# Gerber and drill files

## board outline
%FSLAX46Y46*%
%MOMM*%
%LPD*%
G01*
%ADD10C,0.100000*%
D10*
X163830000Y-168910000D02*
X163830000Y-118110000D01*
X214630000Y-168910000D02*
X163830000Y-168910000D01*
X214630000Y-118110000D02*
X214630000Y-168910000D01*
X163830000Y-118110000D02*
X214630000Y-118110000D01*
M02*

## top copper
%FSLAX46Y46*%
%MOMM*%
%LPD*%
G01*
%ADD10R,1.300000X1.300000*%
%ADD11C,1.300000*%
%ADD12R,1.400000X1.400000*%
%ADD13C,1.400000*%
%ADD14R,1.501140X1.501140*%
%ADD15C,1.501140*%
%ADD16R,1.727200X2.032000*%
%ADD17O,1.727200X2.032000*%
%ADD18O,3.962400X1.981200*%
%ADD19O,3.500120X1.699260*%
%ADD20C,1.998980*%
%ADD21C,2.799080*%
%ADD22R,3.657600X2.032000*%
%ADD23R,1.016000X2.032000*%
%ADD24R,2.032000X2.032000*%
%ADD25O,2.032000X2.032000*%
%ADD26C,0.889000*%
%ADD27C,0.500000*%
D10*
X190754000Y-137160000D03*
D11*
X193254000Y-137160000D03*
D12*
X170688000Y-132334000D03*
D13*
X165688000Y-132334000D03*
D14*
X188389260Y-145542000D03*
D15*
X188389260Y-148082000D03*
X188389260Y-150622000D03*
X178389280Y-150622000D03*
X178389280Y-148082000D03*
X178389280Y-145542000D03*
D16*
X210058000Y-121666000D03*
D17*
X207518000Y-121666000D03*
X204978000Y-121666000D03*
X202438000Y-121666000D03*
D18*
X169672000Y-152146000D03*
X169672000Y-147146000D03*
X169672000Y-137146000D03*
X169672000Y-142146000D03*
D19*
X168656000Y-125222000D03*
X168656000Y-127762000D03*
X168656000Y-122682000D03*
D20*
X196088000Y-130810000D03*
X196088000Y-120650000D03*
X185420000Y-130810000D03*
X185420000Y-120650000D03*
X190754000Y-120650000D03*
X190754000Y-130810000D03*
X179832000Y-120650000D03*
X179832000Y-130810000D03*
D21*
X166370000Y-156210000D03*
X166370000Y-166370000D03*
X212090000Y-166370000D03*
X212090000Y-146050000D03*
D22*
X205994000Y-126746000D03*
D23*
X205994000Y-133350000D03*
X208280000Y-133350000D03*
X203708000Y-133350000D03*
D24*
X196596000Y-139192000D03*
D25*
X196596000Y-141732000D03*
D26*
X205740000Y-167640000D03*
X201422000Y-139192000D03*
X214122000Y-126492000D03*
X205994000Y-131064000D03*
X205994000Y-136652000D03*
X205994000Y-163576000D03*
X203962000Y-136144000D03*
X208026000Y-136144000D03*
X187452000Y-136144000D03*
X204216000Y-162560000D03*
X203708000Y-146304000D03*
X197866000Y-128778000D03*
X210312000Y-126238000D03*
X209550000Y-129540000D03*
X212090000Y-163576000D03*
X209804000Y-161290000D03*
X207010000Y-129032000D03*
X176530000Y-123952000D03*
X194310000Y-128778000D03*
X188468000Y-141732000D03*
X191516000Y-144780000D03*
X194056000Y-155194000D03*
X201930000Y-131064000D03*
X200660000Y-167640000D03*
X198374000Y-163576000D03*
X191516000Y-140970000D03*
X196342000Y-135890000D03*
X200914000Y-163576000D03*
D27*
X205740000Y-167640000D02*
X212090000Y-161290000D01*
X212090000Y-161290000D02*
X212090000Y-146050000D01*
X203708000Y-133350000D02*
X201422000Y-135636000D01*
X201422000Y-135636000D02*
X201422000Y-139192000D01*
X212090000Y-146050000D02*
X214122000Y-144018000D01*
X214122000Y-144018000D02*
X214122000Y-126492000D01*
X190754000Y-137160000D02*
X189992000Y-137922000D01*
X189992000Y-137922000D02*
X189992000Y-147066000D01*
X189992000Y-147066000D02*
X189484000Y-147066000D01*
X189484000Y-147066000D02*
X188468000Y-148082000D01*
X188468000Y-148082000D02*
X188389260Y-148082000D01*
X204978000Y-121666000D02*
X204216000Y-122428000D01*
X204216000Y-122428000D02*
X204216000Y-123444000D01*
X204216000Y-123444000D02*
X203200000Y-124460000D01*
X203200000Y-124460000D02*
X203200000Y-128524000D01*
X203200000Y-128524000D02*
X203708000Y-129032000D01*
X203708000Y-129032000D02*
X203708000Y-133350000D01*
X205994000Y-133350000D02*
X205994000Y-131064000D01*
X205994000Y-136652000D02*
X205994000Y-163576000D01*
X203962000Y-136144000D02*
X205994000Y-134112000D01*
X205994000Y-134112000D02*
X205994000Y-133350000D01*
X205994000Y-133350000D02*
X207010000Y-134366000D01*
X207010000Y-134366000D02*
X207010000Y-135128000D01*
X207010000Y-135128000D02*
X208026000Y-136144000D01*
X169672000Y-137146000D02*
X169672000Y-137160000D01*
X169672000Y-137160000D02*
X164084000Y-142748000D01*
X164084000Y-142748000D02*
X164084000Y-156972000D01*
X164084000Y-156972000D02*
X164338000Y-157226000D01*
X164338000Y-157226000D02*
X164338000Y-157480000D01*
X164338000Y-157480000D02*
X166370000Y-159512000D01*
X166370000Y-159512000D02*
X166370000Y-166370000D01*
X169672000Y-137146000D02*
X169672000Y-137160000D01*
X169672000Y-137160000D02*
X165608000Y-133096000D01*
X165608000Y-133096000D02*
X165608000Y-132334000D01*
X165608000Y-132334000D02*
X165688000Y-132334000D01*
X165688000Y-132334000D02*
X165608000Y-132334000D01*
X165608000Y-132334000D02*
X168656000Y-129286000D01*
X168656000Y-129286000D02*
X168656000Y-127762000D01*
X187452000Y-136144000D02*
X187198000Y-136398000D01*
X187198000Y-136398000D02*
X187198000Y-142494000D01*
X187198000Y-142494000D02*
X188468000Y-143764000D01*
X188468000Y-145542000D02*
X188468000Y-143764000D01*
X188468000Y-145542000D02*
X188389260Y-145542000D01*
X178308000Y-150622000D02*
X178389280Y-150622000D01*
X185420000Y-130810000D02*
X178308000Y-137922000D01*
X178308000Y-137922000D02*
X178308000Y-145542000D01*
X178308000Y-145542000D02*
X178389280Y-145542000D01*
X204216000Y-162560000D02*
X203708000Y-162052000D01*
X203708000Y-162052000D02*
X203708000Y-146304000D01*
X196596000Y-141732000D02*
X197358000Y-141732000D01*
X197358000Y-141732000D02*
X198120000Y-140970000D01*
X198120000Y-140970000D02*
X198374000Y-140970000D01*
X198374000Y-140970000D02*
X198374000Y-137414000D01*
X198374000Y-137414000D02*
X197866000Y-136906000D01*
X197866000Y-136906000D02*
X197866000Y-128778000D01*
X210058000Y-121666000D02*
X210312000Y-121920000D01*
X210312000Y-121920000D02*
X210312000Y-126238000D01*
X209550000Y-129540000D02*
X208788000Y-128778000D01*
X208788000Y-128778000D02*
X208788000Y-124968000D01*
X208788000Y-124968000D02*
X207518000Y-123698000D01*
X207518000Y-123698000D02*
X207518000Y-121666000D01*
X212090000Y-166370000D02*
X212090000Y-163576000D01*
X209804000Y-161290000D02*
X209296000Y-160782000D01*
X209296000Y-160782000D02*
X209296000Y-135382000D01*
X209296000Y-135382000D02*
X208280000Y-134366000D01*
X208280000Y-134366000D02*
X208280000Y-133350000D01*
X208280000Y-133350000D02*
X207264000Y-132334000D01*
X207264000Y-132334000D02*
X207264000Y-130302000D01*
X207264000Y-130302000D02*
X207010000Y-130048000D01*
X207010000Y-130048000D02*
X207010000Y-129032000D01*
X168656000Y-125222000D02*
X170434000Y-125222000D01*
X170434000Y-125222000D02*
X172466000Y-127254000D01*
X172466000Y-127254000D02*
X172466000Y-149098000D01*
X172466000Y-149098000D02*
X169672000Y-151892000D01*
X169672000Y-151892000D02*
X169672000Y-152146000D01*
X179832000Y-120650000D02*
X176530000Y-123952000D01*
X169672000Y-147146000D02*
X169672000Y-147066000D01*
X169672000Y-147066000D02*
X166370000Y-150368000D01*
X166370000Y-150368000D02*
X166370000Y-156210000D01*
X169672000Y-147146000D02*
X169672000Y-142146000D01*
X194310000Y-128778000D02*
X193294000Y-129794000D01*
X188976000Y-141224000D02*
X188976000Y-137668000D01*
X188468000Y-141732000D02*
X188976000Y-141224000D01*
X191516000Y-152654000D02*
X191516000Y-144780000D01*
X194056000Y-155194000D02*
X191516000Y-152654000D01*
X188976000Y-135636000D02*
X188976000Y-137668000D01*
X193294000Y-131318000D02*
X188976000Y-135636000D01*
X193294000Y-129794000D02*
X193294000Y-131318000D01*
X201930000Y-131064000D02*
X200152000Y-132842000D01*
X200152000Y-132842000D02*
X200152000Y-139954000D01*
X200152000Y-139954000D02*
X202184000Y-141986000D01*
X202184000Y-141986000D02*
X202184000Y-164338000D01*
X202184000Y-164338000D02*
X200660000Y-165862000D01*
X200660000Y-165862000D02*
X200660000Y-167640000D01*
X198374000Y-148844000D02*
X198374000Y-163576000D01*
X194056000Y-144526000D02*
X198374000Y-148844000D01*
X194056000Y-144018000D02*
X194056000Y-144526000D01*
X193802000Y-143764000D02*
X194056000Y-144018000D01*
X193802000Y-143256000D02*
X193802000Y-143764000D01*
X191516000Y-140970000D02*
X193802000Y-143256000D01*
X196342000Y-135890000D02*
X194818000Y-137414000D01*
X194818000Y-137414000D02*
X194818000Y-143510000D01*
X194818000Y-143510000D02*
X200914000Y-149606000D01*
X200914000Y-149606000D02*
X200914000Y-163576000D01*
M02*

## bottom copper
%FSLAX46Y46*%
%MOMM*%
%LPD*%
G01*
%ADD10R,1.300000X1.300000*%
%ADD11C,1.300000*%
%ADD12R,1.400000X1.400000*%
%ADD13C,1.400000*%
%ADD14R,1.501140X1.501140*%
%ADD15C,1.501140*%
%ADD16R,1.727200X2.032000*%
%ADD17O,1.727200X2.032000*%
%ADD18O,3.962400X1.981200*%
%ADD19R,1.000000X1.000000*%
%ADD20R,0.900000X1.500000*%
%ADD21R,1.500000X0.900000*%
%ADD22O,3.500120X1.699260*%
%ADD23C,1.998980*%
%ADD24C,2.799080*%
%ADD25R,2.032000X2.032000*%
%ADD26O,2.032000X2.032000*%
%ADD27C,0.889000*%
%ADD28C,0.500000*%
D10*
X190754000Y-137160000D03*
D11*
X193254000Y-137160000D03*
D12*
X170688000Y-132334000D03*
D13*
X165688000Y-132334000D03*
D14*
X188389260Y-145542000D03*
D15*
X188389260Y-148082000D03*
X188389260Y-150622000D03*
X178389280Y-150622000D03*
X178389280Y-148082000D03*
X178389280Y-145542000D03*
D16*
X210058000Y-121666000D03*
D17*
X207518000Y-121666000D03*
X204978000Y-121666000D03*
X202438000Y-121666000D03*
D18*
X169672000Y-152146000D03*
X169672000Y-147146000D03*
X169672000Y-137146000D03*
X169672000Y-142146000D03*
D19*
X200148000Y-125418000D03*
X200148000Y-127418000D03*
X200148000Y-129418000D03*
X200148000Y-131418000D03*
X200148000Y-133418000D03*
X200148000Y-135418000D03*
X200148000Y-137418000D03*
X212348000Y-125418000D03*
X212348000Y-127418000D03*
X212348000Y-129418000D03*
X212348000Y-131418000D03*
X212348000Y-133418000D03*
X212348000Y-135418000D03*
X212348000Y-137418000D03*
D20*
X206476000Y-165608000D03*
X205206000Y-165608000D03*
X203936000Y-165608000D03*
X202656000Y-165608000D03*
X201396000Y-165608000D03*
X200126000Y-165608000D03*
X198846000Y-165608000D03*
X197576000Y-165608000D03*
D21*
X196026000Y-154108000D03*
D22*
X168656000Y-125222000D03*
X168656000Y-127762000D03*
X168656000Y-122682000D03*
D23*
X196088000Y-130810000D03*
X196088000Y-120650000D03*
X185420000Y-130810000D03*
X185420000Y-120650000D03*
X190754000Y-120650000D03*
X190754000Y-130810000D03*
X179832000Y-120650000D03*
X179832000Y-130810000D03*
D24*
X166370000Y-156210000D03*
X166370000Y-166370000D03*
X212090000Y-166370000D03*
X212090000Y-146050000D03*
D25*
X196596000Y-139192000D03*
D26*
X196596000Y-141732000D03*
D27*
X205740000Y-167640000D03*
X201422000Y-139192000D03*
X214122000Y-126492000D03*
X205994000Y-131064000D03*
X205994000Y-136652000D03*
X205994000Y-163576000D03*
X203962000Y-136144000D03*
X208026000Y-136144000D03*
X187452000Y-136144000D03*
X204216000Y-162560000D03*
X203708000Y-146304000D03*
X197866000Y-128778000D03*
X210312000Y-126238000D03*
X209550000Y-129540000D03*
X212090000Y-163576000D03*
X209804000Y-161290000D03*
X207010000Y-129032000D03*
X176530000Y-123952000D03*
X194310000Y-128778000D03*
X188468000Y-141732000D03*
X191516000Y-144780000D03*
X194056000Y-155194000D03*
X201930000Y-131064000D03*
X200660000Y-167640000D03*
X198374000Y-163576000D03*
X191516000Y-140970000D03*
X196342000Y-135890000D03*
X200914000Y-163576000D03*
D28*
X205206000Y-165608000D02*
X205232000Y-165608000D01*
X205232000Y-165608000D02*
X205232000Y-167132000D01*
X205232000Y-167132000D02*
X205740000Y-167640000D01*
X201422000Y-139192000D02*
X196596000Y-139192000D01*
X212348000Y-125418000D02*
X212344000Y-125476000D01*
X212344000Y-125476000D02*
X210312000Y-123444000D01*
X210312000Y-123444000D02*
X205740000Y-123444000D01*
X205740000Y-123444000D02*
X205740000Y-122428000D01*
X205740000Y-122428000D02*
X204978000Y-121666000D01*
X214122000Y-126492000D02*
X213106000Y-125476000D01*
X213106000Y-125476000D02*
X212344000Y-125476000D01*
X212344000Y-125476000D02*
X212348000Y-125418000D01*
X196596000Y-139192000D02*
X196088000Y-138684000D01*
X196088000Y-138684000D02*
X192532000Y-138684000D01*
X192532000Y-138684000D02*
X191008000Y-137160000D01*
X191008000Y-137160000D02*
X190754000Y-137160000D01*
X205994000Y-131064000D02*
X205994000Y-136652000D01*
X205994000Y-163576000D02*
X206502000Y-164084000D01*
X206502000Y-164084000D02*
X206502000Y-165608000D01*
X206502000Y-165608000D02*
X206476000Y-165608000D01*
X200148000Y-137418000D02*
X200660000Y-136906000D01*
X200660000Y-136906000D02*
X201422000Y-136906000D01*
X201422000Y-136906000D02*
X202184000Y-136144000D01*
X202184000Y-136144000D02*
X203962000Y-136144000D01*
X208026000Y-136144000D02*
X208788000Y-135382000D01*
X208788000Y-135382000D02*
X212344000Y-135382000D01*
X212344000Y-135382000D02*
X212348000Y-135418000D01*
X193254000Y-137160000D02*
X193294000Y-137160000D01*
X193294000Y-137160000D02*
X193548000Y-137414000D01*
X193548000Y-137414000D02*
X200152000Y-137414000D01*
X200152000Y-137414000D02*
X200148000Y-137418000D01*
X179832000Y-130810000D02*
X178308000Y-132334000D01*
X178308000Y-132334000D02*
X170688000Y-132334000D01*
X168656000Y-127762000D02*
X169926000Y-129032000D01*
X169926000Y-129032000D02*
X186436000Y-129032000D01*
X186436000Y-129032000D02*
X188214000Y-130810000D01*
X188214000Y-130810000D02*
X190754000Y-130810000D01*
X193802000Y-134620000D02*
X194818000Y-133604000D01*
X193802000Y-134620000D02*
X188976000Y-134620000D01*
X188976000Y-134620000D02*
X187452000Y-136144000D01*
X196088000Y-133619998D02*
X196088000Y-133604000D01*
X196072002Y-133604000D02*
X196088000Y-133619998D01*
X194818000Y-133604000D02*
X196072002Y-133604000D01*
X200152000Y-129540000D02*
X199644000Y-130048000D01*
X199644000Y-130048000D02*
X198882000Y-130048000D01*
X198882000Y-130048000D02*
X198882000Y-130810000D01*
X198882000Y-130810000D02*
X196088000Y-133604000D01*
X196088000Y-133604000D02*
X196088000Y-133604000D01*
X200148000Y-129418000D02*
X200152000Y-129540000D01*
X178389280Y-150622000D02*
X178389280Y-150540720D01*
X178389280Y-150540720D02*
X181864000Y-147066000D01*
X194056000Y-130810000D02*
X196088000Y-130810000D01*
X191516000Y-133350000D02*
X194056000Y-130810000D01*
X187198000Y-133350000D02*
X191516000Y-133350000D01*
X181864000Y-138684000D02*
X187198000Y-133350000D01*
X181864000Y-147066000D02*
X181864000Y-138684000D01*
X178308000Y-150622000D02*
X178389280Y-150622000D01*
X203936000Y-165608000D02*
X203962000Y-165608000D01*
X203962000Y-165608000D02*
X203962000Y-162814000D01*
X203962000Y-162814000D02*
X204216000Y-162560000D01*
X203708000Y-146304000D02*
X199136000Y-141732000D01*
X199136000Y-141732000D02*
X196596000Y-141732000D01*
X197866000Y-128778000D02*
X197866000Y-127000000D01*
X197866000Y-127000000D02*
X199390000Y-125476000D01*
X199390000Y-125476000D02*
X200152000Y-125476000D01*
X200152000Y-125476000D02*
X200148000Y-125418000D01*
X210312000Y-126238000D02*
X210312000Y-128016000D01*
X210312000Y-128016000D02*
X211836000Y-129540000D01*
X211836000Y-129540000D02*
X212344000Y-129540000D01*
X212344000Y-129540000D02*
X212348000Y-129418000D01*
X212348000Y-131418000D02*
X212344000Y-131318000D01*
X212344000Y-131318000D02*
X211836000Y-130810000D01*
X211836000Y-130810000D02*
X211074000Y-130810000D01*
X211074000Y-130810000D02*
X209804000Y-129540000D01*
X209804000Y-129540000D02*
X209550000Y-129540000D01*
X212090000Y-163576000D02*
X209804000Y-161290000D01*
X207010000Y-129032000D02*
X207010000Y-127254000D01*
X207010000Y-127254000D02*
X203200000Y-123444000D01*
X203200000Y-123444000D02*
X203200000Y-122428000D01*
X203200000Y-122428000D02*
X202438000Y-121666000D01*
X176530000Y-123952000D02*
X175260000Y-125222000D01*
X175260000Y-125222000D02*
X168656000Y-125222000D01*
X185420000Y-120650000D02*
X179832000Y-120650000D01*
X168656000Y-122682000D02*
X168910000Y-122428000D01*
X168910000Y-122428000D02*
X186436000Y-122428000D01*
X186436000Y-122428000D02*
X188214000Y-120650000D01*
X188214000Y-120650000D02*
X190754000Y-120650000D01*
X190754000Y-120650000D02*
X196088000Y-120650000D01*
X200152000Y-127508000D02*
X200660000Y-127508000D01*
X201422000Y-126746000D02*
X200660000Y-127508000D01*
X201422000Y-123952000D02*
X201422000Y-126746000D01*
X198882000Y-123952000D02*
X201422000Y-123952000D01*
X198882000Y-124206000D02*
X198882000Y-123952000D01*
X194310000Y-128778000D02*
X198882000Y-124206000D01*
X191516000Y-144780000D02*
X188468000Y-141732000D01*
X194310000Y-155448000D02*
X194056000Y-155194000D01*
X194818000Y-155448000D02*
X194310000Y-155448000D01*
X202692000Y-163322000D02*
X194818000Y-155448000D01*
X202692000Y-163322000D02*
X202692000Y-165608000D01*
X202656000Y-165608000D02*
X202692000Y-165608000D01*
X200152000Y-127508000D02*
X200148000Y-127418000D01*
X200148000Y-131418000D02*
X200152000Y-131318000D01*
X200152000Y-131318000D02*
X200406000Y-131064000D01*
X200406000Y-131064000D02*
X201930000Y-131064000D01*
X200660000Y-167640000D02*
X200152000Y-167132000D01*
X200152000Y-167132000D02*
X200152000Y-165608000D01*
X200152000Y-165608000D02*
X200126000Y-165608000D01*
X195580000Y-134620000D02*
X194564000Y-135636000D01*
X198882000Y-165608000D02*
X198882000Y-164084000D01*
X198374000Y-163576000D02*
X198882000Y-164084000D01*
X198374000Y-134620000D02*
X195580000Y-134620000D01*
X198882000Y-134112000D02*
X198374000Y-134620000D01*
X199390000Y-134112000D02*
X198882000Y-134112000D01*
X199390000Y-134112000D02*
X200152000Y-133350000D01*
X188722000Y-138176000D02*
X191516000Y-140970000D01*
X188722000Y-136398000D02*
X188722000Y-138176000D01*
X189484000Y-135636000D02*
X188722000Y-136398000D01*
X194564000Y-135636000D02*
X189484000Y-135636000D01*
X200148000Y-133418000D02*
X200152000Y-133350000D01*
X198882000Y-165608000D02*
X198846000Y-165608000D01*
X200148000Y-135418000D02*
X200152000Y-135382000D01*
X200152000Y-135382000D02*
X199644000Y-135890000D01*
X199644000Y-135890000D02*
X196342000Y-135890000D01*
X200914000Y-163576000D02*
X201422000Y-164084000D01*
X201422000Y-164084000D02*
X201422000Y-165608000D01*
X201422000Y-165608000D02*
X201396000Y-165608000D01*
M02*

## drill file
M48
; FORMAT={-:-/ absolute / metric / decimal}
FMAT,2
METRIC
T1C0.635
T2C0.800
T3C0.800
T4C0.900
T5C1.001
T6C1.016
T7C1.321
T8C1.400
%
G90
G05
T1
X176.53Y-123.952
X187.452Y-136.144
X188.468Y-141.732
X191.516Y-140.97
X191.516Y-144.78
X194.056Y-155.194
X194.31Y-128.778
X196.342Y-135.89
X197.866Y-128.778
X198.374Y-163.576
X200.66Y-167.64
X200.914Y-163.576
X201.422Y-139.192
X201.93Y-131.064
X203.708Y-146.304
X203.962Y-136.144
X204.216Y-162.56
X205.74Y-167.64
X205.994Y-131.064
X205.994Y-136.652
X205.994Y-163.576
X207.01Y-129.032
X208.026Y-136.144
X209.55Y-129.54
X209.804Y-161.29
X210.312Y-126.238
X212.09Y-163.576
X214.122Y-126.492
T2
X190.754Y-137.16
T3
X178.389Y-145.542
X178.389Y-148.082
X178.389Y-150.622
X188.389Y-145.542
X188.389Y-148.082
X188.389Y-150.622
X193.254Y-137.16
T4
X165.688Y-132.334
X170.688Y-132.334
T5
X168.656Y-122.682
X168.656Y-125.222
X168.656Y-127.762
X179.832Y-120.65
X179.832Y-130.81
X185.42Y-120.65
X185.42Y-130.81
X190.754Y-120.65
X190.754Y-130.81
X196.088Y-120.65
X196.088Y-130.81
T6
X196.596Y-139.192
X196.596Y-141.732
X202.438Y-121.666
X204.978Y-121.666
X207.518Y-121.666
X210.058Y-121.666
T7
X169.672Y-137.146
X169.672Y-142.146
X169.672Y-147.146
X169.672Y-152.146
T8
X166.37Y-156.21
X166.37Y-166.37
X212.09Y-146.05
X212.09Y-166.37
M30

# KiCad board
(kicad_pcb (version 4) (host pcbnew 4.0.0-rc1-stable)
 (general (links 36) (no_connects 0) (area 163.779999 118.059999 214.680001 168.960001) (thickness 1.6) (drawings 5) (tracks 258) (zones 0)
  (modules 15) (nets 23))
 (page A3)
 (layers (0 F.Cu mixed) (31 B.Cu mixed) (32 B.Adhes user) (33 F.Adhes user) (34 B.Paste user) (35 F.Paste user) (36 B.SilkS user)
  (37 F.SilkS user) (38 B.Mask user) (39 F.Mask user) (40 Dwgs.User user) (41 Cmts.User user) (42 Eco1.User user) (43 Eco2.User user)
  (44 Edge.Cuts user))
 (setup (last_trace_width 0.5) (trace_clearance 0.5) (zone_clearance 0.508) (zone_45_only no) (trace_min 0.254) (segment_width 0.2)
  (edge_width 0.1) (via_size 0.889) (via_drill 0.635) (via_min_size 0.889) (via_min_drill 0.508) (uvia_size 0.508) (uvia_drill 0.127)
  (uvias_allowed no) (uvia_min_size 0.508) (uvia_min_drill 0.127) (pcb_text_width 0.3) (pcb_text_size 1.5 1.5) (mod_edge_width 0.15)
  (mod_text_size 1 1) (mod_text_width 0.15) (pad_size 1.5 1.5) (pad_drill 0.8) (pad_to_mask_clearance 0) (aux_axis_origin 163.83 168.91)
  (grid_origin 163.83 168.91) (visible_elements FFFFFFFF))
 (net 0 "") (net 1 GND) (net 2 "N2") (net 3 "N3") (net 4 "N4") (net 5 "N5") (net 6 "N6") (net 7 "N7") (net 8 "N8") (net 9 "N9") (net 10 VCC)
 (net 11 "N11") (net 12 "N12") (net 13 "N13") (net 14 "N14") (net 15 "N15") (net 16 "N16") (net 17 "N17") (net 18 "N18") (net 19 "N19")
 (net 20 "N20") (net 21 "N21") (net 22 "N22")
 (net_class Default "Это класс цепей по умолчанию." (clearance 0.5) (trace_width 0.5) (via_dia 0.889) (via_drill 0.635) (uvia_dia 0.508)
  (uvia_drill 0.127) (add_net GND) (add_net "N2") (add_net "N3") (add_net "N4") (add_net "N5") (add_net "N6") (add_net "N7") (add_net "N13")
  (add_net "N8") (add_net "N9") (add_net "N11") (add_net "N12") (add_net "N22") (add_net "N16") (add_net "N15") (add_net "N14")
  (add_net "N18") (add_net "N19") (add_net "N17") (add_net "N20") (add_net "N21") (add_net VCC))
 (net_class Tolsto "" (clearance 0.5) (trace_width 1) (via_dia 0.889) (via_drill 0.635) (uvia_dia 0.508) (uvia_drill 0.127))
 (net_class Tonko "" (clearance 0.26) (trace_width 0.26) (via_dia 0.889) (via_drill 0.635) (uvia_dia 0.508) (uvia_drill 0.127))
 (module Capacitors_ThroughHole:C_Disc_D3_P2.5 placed (layer B.Cu) (at 190.754 137.16)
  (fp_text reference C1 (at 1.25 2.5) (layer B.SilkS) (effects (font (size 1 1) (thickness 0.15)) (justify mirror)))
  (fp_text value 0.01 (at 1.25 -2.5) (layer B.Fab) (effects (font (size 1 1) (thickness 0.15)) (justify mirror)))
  (pad 1 thru_hole rect (at 0 0) (size 1.3 1.3) (drill 0.8) (layers *.Cu *.Mask B.SilkS) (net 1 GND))
  (pad 2 thru_hole circle (at 2.5 0) (size 1.3 1.3) (drill 0.8001) (layers *.Cu *.Mask B.SilkS) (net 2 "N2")))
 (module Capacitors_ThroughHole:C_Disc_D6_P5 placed (layer F.Cu) (at 170.688 132.334 180)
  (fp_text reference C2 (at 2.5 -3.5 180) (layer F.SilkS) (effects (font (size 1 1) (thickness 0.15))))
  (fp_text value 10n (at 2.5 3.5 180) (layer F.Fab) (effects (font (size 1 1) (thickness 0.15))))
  (pad 1 thru_hole rect (at 0 0 180) (size 1.4 1.4) (drill 0.9) (layers *.Cu *.Mask F.SilkS) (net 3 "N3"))
  (pad 2 thru_hole circle (at 5 0 180) (size 1.4 1.4) (drill 0.9) (layers *.Cu *.Mask F.SilkS) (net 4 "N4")))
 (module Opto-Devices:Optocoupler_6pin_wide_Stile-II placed (layer B.Cu) (at 183.388 148.082 270)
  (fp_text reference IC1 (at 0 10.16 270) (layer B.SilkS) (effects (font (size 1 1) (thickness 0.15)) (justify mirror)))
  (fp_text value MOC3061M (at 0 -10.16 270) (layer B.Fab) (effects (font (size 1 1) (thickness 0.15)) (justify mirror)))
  (pad 1 thru_hole rect (at -2.54 -5.00126 270) (size 1.50114 1.50114) (drill 0.8001) (layers *.Cu *.Mask B.SilkS) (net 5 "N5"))
  (pad 2 thru_hole circle (at 0 -5.00126 270) (size 1.50114 1.50114) (drill 0.8001) (layers *.Cu *.Mask B.SilkS) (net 1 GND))
  (pad 3 thru_hole circle (at 2.54 -5.00126 270) (size 1.50114 1.50114) (drill 0.8001) (layers *.Cu *.Mask B.SilkS))
  (pad 4 thru_hole circle (at 2.54 4.99872 270) (size 1.50114 1.50114) (drill 0.8001) (layers *.Cu *.Mask B.SilkS) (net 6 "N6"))
  (pad 5 thru_hole circle (at 0 4.99872 270) (size 1.50114 1.50114) (drill 0.8001) (layers *.Cu *.Mask B.SilkS))
  (pad 6 thru_hole circle (at -2.54 4.99872 270) (size 1.50114 1.50114) (drill 0.8001) (layers *.Cu *.Mask B.SilkS) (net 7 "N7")))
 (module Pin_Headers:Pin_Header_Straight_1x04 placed (layer F.Cu) (at 210.058 121.666 270)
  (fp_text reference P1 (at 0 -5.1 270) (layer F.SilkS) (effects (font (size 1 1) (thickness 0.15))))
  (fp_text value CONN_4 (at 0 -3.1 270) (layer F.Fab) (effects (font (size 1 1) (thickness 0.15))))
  (pad 1 thru_hole rect (at 0 0 270) (size 2.032 1.7272) (drill 1.016) (layers *.Cu *.Mask F.SilkS) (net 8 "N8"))
  (pad 2 thru_hole oval (at 0 2.54 270) (size 2.032 1.7272) (drill 1.016) (layers *.Cu *.Mask F.SilkS) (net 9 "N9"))
  (pad 3 thru_hole oval (at 0 5.08 270) (size 2.032 1.7272) (drill 1.016) (layers *.Cu *.Mask F.SilkS) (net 1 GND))
  (pad 4 thru_hole oval (at 0 7.62 270) (size 2.032 1.7272) (drill 1.016) (layers *.Cu *.Mask F.SilkS) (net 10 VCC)))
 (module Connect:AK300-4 (layer B.Cu) (at 169.672 152.146 90)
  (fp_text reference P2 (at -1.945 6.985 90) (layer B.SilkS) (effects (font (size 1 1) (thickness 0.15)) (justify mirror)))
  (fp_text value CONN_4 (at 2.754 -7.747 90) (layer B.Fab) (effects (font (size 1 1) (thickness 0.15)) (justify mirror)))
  (pad 1 thru_hole oval (at 0 0 90) (size 1.9812 3.9624) (drill 1.3208) (layers *.Cu B.Paste B.SilkS B.Mask) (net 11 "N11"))
  (pad 2 thru_hole oval (at 5 0 90) (size 1.9812 3.9624) (drill 1.3208) (layers *.Cu B.Paste B.SilkS B.Mask) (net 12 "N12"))
  (pad 4 thru_hole oval (at 15 0 90) (size 1.9812 3.9624) (drill 1.3208) (layers *.Cu B.Paste B.SilkS B.Mask) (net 4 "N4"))
  (pad 3 thru_hole oval (at 10 0 90) (size 1.9812 3.9624) (drill 1.3208) (layers *.Cu *.Mask B.SilkS) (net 12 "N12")))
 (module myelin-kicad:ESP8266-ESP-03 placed (layer B.Cu) (at 206.248 131.318)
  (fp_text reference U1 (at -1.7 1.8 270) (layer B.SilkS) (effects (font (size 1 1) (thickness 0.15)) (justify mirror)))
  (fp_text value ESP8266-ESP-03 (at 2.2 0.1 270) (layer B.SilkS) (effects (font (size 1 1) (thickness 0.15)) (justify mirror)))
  (pad 14 smd rect (at -6.1 -5.9) (size 1 1) (layers B.Cu B.Paste B.Mask) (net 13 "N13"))
  (pad 13 smd rect (at -6.1 -3.9) (size 1 1) (layers B.Cu B.Paste B.Mask) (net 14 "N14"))
  (pad 12 smd rect (at -6.1 -1.9) (size 1 1) (layers B.Cu B.Paste B.Mask) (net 5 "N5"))
  (pad 11 smd rect (at -6.1 0.1) (size 1 1) (layers B.Cu B.Paste B.Mask) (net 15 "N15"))
  (pad 10 smd rect (at -6.1 2.1) (size 1 1) (layers B.Cu B.Paste B.Mask) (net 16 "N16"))
  (pad 9 smd rect (at -6.1 4.1) (size 1 1) (layers B.Cu B.Paste B.Mask) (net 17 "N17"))
  (pad 8 smd rect (at -6.1 6.1) (size 1 1) (layers B.Cu B.Paste B.Mask) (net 2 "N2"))
  (pad 1 smd rect (at 6.1 -5.9) (size 1 1) (layers B.Cu B.Paste B.Mask) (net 1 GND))
  (pad 2 smd rect (at 6.1 -3.9) (size 1 1) (layers B.Cu B.Paste B.Mask))
  (pad 3 smd rect (at 6.1 -1.9) (size 1 1) (layers B.Cu B.Paste B.Mask) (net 8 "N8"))
  (pad 4 smd rect (at 6.1 0.1) (size 1 1) (layers B.Cu B.Paste B.Mask) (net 9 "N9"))
  (pad 5 smd rect (at 6.1 2.1) (size 1 1) (layers B.Cu B.Paste B.Mask) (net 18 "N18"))
  (pad 6 smd rect (at 6.1 4.1) (size 1 1) (layers B.Cu B.Paste B.Mask) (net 2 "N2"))
  (pad 7 smd rect (at 6.1 6.1) (size 1 1) (layers B.Cu B.Paste B.Mask) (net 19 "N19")))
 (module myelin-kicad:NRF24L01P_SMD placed (layer B.Cu) (at 208.026 165.608 90)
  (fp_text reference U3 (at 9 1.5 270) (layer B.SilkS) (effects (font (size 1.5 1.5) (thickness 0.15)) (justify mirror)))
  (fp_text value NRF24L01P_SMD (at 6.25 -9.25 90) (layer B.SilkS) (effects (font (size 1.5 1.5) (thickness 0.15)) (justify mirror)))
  (pad 1 smd rect (at 0 -1.55 90) (size 1.5 0.9) (layers B.Cu B.Paste B.Mask) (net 2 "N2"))
  (pad 2 smd rect (at 0 -2.82 90) (size 1.5 0.9) (layers B.Cu B.Paste B.Mask) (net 1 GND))
  (pad 3 smd rect (at 0 -4.09 90) (size 1.5 0.9) (layers B.Cu B.Paste B.Mask) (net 13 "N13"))
  (pad 4 smd rect (at 0 -5.37 90) (size 1.5 0.9) (layers B.Cu B.Paste B.Mask) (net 14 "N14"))
  (pad 5 smd rect (at 0 -6.63 90) (size 1.5 0.9) (layers B.Cu B.Paste B.Mask) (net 17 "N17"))
  (pad 6 smd rect (at 0 -7.9 90) (size 1.5 0.9) (layers B.Cu B.Paste B.Mask) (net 15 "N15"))
  (pad 7 smd rect (at 0 -9.18 90) (size 1.5 0.9) (layers B.Cu B.Paste B.Mask) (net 16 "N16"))
  (pad 8 smd rect (at 0 -10.45 90) (size 1.5 0.9) (layers B.Cu B.Paste B.Mask) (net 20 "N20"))
  (pad 9 smd rect (at 11.5 -12 90) (size 0.9 1.5) (layers B.Cu B.Paste B.Mask) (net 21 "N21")))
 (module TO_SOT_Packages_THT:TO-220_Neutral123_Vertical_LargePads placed (layer F.Cu) (at 168.656 125.222 90)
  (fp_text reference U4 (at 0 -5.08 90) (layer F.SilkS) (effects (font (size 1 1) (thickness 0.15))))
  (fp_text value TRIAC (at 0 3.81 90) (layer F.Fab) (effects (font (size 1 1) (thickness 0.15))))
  (pad 2 thru_hole oval (at 0 0 180) (size 3.50012 1.69926) (drill 1.00076) (layers *.Cu *.Mask F.SilkS) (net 11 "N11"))
  (pad 1 thru_hole oval (at -2.54 0 180) (size 3.50012 1.69926) (drill 1.00076) (layers *.Cu *.Mask F.SilkS) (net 4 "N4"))
  (pad 3 thru_hole oval (at 2.54 0 180) (size 3.50012 1.69926) (drill 1.00076) (layers *.Cu *.Mask F.SilkS) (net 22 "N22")))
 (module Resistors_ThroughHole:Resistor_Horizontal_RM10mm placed (layer F.Cu) (at 196.088 125.73 90)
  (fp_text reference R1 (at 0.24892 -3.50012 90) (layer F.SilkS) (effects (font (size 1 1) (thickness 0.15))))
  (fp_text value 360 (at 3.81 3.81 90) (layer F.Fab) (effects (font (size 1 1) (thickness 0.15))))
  (pad 1 thru_hole circle (at -5.08 0 90) (size 1.99898 1.99898) (drill 1.00076) (layers *.Cu *.SilkS *.Mask) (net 6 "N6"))
  (pad 2 thru_hole circle (at 5.08 0 90) (size 1.99898 1.99898) (drill 1.00076) (layers *.Cu *.SilkS *.Mask) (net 22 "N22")))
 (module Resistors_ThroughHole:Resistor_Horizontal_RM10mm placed (layer F.Cu) (at 185.42 125.73 90)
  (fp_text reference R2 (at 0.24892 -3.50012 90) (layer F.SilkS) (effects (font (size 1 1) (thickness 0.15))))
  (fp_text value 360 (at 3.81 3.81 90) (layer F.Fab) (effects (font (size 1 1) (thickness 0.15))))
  (pad 1 thru_hole circle (at -5.08 0 90) (size 1.99898 1.99898) (drill 1.00076) (layers *.Cu *.SilkS *.Mask) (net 7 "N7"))
  (pad 2 thru_hole circle (at 5.08 0 90) (size 1.99898 1.99898) (drill 1.00076) (layers *.Cu *.SilkS *.Mask) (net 11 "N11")))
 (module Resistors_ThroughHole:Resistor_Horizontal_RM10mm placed (layer F.Cu) (at 190.754 125.73 270)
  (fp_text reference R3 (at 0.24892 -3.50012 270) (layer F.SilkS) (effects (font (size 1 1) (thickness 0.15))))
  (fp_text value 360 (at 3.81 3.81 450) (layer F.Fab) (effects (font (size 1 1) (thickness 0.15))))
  (pad 1 thru_hole circle (at -5.08 0 270) (size 1.99898 1.99898) (drill 1.00076) (layers *.Cu *.SilkS *.Mask) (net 22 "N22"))
  (pad 2 thru_hole circle (at 5.08 0 270) (size 1.99898 1.99898) (drill 1.00076) (layers *.Cu *.SilkS *.Mask) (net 4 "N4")))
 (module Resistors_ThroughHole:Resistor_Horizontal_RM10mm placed (layer F.Cu) (at 179.832 125.73 270)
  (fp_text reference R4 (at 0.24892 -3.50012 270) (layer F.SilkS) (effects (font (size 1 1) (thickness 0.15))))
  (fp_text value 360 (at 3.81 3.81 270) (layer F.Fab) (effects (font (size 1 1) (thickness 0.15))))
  (pad 1 thru_hole circle (at -5.08 0 270) (size 1.99898 1.99898) (drill 1.00076) (layers *.Cu *.SilkS *.Mask) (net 11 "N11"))
  (pad 2 thru_hole circle (at 5.08 0 270) (size 1.99898 1.99898) (drill 1.00076) (layers *.Cu *.SilkS *.Mask) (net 3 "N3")))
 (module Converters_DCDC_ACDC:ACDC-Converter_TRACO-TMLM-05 (layer F.Cu) (at 166.37 156.21)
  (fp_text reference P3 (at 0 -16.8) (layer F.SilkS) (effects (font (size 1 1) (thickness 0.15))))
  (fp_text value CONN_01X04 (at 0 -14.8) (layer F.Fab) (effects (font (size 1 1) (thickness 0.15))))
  (pad 1 thru_hole circle (at 0 0) (size 2.79908 2.79908) (drill 1.39954) (layers *.Cu *.Mask F.SilkS) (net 12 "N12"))
  (pad 2 thru_hole circle (at 0 10.16) (size 2.79908 2.79908) (drill 1.39954) (layers *.Cu *.Mask F.SilkS) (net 4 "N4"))
  (pad 3 thru_hole circle (at 45.72 10.16) (size 2.79908 2.79908) (drill 1.39954) (layers *.Cu *.Mask F.SilkS) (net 10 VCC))
  (pad 4 thru_hole circle (at 45.72 -10.16) (size 2.79908 2.79908) (drill 1.39954) (layers *.Cu *.Mask F.SilkS) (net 1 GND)))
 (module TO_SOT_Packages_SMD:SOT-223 (layer F.Cu) (at 205.994 130.048)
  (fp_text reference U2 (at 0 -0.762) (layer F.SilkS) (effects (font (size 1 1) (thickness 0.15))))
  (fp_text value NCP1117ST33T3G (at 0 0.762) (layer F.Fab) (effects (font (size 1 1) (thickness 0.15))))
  (pad 4 smd rect (at 0 -3.302) (size 3.6576 2.032) (layers F.Cu F.Paste F.Mask))
  (pad 2 smd rect (at 0 3.302) (size 1.016 2.032) (layers F.Cu F.Paste F.Mask) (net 2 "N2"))
  (pad 3 smd rect (at 2.286 3.302) (size 1.016 2.032) (layers F.Cu F.Paste F.Mask) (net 10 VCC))
  (pad 1 smd rect (at -2.286 3.302) (size 1.016 2.032) (layers F.Cu F.Paste F.Mask) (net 1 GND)))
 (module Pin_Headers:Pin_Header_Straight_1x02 (layer F.Cu) (at 196.596 139.192)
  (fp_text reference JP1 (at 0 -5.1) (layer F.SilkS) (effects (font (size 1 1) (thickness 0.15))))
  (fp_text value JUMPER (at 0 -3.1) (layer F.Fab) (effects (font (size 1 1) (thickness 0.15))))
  (pad 1 thru_hole rect (at 0 0) (size 2.032 2.032) (drill 1.016) (layers *.Cu *.Mask F.SilkS) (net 1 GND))
  (pad 2 thru_hole oval (at 0 2.54) (size 2.032 2.032) (drill 1.016) (layers *.Cu *.Mask F.SilkS) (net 13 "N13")))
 (gr_line (start 163.83 168.91) (end 163.83 118.11) (angle 90) (layer Edge.Cuts) (width 0.1))
 (gr_line (start 214.63 168.91) (end 163.83 168.91) (angle 90) (layer Edge.Cuts) (width 0.1))
 (gr_line (start 214.63 118.11) (end 214.63 168.91) (angle 90) (layer Edge.Cuts) (width 0.1))
 (gr_line (start 163.83 118.11) (end 214.63 118.11) (angle 90) (layer Edge.Cuts) (width 0.1))
 (segment (start 205.206 165.608) (end 205.232 165.608) (width 0.5) (layer B.Cu) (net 1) (status 80000))
 (segment (start 205.232 165.608) (end 205.232 167.132) (width 0.5) (layer B.Cu) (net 1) (status 80000))
 (segment (start 205.232 167.132) (end 205.74 167.64) (width 0.5) (layer B.Cu) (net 1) (status 80000))
 (segment (start 205.74 167.64) (end 212.09 161.29) (width 0.5) (layer F.Cu) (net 1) (status 80000))
 (segment (start 212.09 161.29) (end 212.09 146.05) (width 0.5) (layer F.Cu) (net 1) (status 80000))
 (segment (start 203.708 133.35) (end 201.422 135.636) (width 0.5) (layer F.Cu) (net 1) (status 80000))
 (segment (start 201.422 135.636) (end 201.422 139.192) (width 0.5) (layer F.Cu) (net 1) (status 80000))
 (segment (start 201.422 139.192) (end 196.596 139.192) (width 0.5) (layer B.Cu) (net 1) (status 80000))
 (segment (start 212.348 125.418) (end 212.344 125.476) (width 0.5) (layer B.Cu) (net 1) (status 80000))
 (segment (start 212.344 125.476) (end 210.312 123.444) (width 0.5) (layer B.Cu) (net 1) (status 80000))
 (segment (start 210.312 123.444) (end 205.74 123.444) (width 0.5) (layer B.Cu) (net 1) (status 80000))
 (segment (start 205.74 123.444) (end 205.74 122.428) (width 0.5) (layer B.Cu) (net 1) (status 80000))
 (segment (start 205.74 122.428) (end 204.978 121.666) (width 0.5) (layer B.Cu) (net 1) (status 80000))
 (segment (start 212.09 146.05) (end 214.122 144.018) (width 0.5) (layer F.Cu) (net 1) (status 80000))
 (segment (start 214.122 144.018) (end 214.122 126.492) (width 0.5) (layer F.Cu) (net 1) (status 80000))
 (segment (start 214.122 126.492) (end 213.106 125.476) (width 0.5) (layer B.Cu) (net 1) (status 80000))
 (segment (start 213.106 125.476) (end 212.344 125.476) (width 0.5) (layer B.Cu) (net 1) (status 80000))
 (segment (start 212.344 125.476) (end 212.348 125.418) (width 0.5) (layer B.Cu) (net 1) (status 80000))
 (segment (start 190.754 137.16) (end 189.992 137.922) (width 0.5) (layer F.Cu) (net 1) (status 80000))
 (segment (start 189.992 137.922) (end 189.992 147.066) (width 0.5) (layer F.Cu) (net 1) (status 80000))
 (segment (start 189.992 147.066) (end 189.484 147.066) (width 0.5) (layer F.Cu) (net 1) (status 80000))
 (segment (start 189.484 147.066) (end 188.468 148.082) (width 0.5) (layer F.Cu) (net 1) (status 80000))
 (segment (start 188.468 148.082) (end 188.38926 148.082) (width 0.5) (layer F.Cu) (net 1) (status 80000))
 (segment (start 204.978 121.666) (end 204.216 122.428) (width 0.5) (layer F.Cu) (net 1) (status 80000))
 (segment (start 204.216 122.428) (end 204.216 123.444) (width 0.5) (layer F.Cu) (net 1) (status 80000))
 (segment (start 204.216 123.444) (end 203.2 124.46) (width 0.5) (layer F.Cu) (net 1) (status 80000))
 (segment (start 203.2 124.46) (end 203.2 128.524) (width 0.5) (layer F.Cu) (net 1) (status 80000))
 (segment (start 203.2 128.524) (end 203.708 129.032) (width 0.5) (layer F.Cu) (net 1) (status 80000))
 (segment (start 203.708 129.032) (end 203.708 133.35) (width 0.5) (layer F.Cu) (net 1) (status 80000))
 (segment (start 196.596 139.192) (end 196.088 138.684) (width 0.5) (layer B.Cu) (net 1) (status 80000))
 (segment (start 196.088 138.684) (end 192.532 138.684) (width 0.5) (layer B.Cu) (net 1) (status 80000))
 (segment (start 192.532 138.684) (end 191.008 137.16) (width 0.5) (layer B.Cu) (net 1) (status 80000))
 (segment (start 191.008 137.16) (end 190.754 137.16) (width 0.5) (layer B.Cu) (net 1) (status 80000))
 (segment (start 205.994 133.35) (end 205.994 131.064) (width 0.5) (layer F.Cu) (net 2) (status 80000))
 (segment (start 205.994 131.064) (end 205.994 136.652) (width 0.5) (layer B.Cu) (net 2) (status 80000))
 (segment (start 205.994 136.652) (end 205.994 163.576) (width 0.5) (layer F.Cu) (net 2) (status 80000))
 (segment (start 205.994 163.576) (end 206.502 164.084) (width 0.5) (layer B.Cu) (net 2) (status 80000))
 (segment (start 206.502 164.084) (end 206.502 165.608) (width 0.5) (layer B.Cu) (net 2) (status 80000))
 (segment (start 206.502 165.608) (end 206.476 165.608) (width 0.5) (layer B.Cu) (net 2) (status 80000))
 (segment (start 200.148 137.418) (end 200.66 136.906) (width 0.5) (layer B.Cu) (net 2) (status 80000))
 (segment (start 200.66 136.906) (end 201.422 136.906) (width 0.5) (layer B.Cu) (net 2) (status 80000))
 (segment (start 201.422 136.906) (end 202.184 136.144) (width 0.5) (layer B.Cu) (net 2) (status 80000))
 (segment (start 202.184 136.144) (end 203.962 136.144) (width 0.5) (layer B.Cu) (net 2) (status 80000))
 (segment (start 203.962 136.144) (end 205.994 134.112) (width 0.5) (layer F.Cu) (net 2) (status 80000))
 (segment (start 205.994 134.112) (end 205.994 133.35) (width 0.5) (layer F.Cu) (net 2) (status 80000))
 (segment (start 205.994 133.35) (end 207.01 134.366) (width 0.5) (layer F.Cu) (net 2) (status 80000))
 (segment (start 207.01 134.366) (end 207.01 135.128) (width 0.5) (layer F.Cu) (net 2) (status 80000))
 (segment (start 207.01 135.128) (end 208.026 136.144) (width 0.5) (layer F.Cu) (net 2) (status 80000))
 (segment (start 208.026 136.144) (end 208.788 135.382) (width 0.5) (layer B.Cu) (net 2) (status 80000))
 (segment (start 208.788 135.382) (end 212.344 135.382) (width 0.5) (layer B.Cu) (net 2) (status 80000))
 (segment (start 212.344 135.382) (end 212.348 135.418) (width 0.5) (layer B.Cu) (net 2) (status 80000))
 (segment (start 193.254 137.16) (end 193.294 137.16) (width 0.5) (layer B.Cu) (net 2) (status 80000))
 (segment (start 193.294 137.16) (end 193.548 137.414) (width 0.5) (layer B.Cu) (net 2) (status 80000))
 (segment (start 193.548 137.414) (end 200.152 137.414) (width 0.5) (layer B.Cu) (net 2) (status 80000))
 (segment (start 200.152 137.414) (end 200.148 137.418) (width 0.5) (layer B.Cu) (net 2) (status 80000))
 (segment (start 179.832 130.81) (end 178.308 132.334) (width 0.5) (layer B.Cu) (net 3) (status 80000))
 (segment (start 178.308 132.334) (end 170.688 132.334) (width 0.5) (layer B.Cu) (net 3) (status 80000))
 (segment (start 169.672 137.146) (end 169.672 137.16) (width 0.5) (layer F.Cu) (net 4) (status 80000))
 (segment (start 169.672 137.16) (end 164.084 142.748) (width 0.5) (layer F.Cu) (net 4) (status 80000))
 (segment (start 164.084 142.748) (end 164.084 156.972) (width 0.5) (layer F.Cu) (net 4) (status 80000))
 (segment (start 164.084 156.972) (end 164.338 157.226) (width 0.5) (layer F.Cu) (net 4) (status 80000))
 (segment (start 164.338 157.226) (end 164.338 157.48) (width 0.5) (layer F.Cu) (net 4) (status 80000))
 (segment (start 164.338 157.48) (end 166.37 159.512) (width 0.5) (layer F.Cu) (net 4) (status 80000))
 (segment (start 166.37 159.512) (end 166.37 166.37) (width 0.5) (layer F.Cu) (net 4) (status 80000))
 (segment (start 168.656 127.762) (end 169.926 129.032) (width 0.5) (layer B.Cu) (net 4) (status 80000))
 (segment (start 169.926 129.032) (end 186.436 129.032) (width 0.5) (layer B.Cu) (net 4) (status 80000))
 (segment (start 186.436 129.032) (end 188.214 130.81) (width 0.5) (layer B.Cu) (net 4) (status 80000))
 (segment (start 188.214 130.81) (end 190.754 130.81) (width 0.5) (layer B.Cu) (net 4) (status 80000))
 (segment (start 169.672 137.146) (end 169.672 137.16) (width 0.5) (layer F.Cu) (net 4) (status 80000))
 (segment (start 169.672 137.16) (end 165.608 133.096) (width 0.5) (layer F.Cu) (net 4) (status 80000))
 (segment (start 165.608 133.096) (end 165.608 132.334) (width 0.5) (layer F.Cu) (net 4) (status 80000))
 (segment (start 165.608 132.334) (end 165.688 132.334) (width 0.5) (layer F.Cu) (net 4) (status 80000))
 (segment (start 165.688 132.334) (end 165.608 132.334) (width 0.5) (layer F.Cu) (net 4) (status 80000))
 (segment (start 165.608 132.334) (end 168.656 129.286) (width 0.5) (layer F.Cu) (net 4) (status 80000))
 (segment (start 168.656 129.286) (end 168.656 127.762) (width 0.5) (layer F.Cu) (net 4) (status 80000))
 (segment (start 193.802 134.62) (end 194.818 133.604) (width 0.5) (layer B.Cu) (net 5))
 (segment (start 193.802 134.62) (end 188.976 134.62) (width 0.5) (layer B.Cu) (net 5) (status 80000))
 (segment (start 188.976 134.62) (end 187.452 136.144) (width 0.5) (layer B.Cu) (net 5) (status 80000))
 (segment (start 187.452 136.144) (end 187.198 136.398) (width 0.5) (layer F.Cu) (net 5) (status 80000))
 (segment (start 187.198 136.398) (end 187.198 142.494) (width 0.5) (layer F.Cu) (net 5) (status 80000))
 (segment (start 187.198 142.494) (end 188.468 143.764) (width 0.5) (layer F.Cu) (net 5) (status 80000))
 (segment (start 188.468 145.542) (end 188.468 143.764) (width 0.5) (layer F.Cu) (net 5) (status 80000))
 (segment (start 196.088 133.619998) (end 196.088 133.604) (width 0.5) (layer B.Cu) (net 5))
 (segment (start 196.072002 133.604) (end 196.088 133.619998) (width 0.5) (layer B.Cu) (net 5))
 (segment (start 194.818 133.604) (end 196.072002 133.604) (width 0.5) (layer B.Cu) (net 5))
 (segment (start 200.152 129.54) (end 199.644 130.048) (width 0.5) (layer B.Cu) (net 5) (status 80000))
 (segment (start 199.644 130.048) (end 198.882 130.048) (width 0.5) (layer B.Cu) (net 5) (status 80000))
 (segment (start 198.882 130.048) (end 198.882 130.81) (width 0.5) (layer B.Cu) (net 5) (status 80000))
 (segment (start 198.882 130.81) (end 196.088 133.604) (width 0.5) (layer B.Cu) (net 5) (status 80000))
 (segment (start 196.088 133.604) (end 196.088 133.604) (width 0.5) (layer B.Cu) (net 5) (status 80000))
 (segment (start 200.148 129.418) (end 200.152 129.54) (width 0.5) (layer B.Cu) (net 5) (status 80000))
 (segment (start 188.468 145.542) (end 188.38926 145.542) (width 0.5) (layer F.Cu) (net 5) (status 80000))
 (segment (start 178.38928 150.622) (end 178.38928 150.54072) (width 0.5) (layer B.Cu) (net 6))
 (segment (start 178.38928 150.54072) (end 181.864 147.066) (width 0.5) (layer B.Cu) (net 6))
 (segment (start 194.056 130.81) (end 196.088 130.81) (width 0.5) (layer B.Cu) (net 6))
 (segment (start 191.516 133.35) (end 194.056 130.81) (width 0.5) (layer B.Cu) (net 6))
 (segment (start 187.198 133.35) (end 191.516 133.35) (width 0.5) (layer B.Cu) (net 6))
 (segment (start 181.864 138.684) (end 187.198 133.35) (width 0.5) (layer B.Cu) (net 6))
 (segment (start 181.864 147.066) (end 181.864 138.684) (width 0.5) (layer B.Cu) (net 6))
 (segment (start 178.308 150.622) (end 178.38928 150.622) (width 0.5) (layer B.Cu) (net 6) (status 80000))
 (segment (start 178.308 150.622) (end 178.38928 150.622) (width 0.5) (layer F.Cu) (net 6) (status 80000))
 (segment (start 185.42 130.81) (end 178.308 137.922) (width 0.5) (layer F.Cu) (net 7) (status 80000))
 (segment (start 178.308 137.922) (end 178.308 145.542) (width 0.5) (layer F.Cu) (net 7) (status 80000))
 (segment (start 178.308 145.542) (end 178.38928 145.542) (width 0.5) (layer F.Cu) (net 7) (status 80000))
 (segment (start 203.936 165.608) (end 203.962 165.608) (width 0.5) (layer B.Cu) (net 13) (status 80000))
 (segment (start 203.962 165.608) (end 203.962 162.814) (width 0.5) (layer B.Cu) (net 13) (status 80000))
 (segment (start 203.962 162.814) (end 204.216 162.56) (width 0.5) (layer B.Cu) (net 13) (status 80000))
 (segment (start 204.216 162.56) (end 203.708 162.052) (width 0.5) (layer F.Cu) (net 13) (status 80000))
 (segment (start 203.708 162.052) (end 203.708 146.304) (width 0.5) (layer F.Cu) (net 13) (status 80000))
 (segment (start 203.708 146.304) (end 199.136 141.732) (width 0.5) (layer B.Cu) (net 13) (status 80000))
 (segment (start 199.136 141.732) (end 196.596 141.732) (width 0.5) (layer B.Cu) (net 13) (status 80000))
 (segment (start 196.596 141.732) (end 197.358 141.732) (width 0.5) (layer F.Cu) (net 13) (status 80000))
 (segment (start 197.358 141.732) (end 198.12 140.97) (width 0.5) (layer F.Cu) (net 13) (status 80000))
 (segment (start 198.12 140.97) (end 198.374 140.97) (width 0.5) (layer F.Cu) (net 13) (status 80000))
 (segment (start 198.374 140.97) (end 198.374 137.414) (width 0.5) (layer F.Cu) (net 13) (status 80000))
 (segment (start 198.374 137.414) (end 197.866 136.906) (width 0.5) (layer F.Cu) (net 13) (status 80000))
 (segment (start 197.866 136.906) (end 197.866 128.778) (width 0.5) (layer F.Cu) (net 13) (status 80000))
 (segment (start 197.866 128.778) (end 197.866 127) (width 0.5) (layer B.Cu) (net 13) (status 80000))
 (segment (start 197.866 127) (end 199.39 125.476) (width 0.5) (layer B.Cu) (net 13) (status 80000))
 (segment (start 199.39 125.476) (end 200.152 125.476) (width 0.5) (layer B.Cu) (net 13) (status 80000))
 (segment (start 200.152 125.476) (end 200.148 125.418) (width 0.5) (layer B.Cu) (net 13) (status 80000))
 (segment (start 210.058 121.666) (end 210.312 121.92) (width 0.5) (layer F.Cu) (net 8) (status 80000))
 (segment (start 210.312 121.92) (end 210.312 126.238) (width 0.5) (layer F.Cu) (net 8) (status 80000))
 (segment (start 210.312 126.238) (end 210.312 128.016) (width 0.5) (layer B.Cu) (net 8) (status 80000))
 (segment (start 210.312 128.016) (end 211.836 129.54) (width 0.5) (layer B.Cu) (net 8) (status 80000))
 (segment (start 211.836 129.54) (end 212.344 129.54) (width 0.5) (layer B.Cu) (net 8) (status 80000))
 (segment (start 212.344 129.54) (end 212.348 129.418) (width 0.5) (layer B.Cu) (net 8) (status 80000))
 (segment (start 212.348 131.418) (end 212.344 131.318) (width 0.5) (layer B.Cu) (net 9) (status 80000))
 (segment (start 212.344 131.318) (end 211.836 130.81) (width 0.5) (layer B.Cu) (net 9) (status 80000))
 (segment (start 211.836 130.81) (end 211.074 130.81) (width 0.5) (layer B.Cu) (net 9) (status 80000))
 (segment (start 211.074 130.81) (end 209.804 129.54) (width 0.5) (layer B.Cu) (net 9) (status 80000))
 (segment (start 209.804 129.54) (end 209.55 129.54) (width 0.5) (layer B.Cu) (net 9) (status 80000))
 (segment (start 209.55 129.54) (end 208.788 128.778) (width 0.5) (layer F.Cu) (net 9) (status 80000))
 (segment (start 208.788 128.778) (end 208.788 124.968) (width 0.5) (layer F.Cu) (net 9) (status 80000))
 (segment (start 208.788 124.968) (end 207.518 123.698) (width 0.5) (layer F.Cu) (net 9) (status 80000))
 (segment (start 207.518 123.698) (end 207.518 121.666) (width 0.5) (layer F.Cu) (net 9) (status 80000))
 (segment (start 212.09 166.37) (end 212.09 163.576) (width 0.5) (layer F.Cu) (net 10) (status 80000))
 (segment (start 212.09 163.576) (end 209.804 161.29) (width 0.5) (layer B.Cu) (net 10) (status 80000))
 (segment (start 209.804 161.29) (end 209.296 160.782) (width 0.5) (layer F.Cu) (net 10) (status 80000))
 (segment (start 209.296 160.782) (end 209.296 135.382) (width 0.5) (layer F.Cu) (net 10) (status 80000))
 (segment (start 209.296 135.382) (end 208.28 134.366) (width 0.5) (layer F.Cu) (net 10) (status 80000))
 (segment (start 208.28 134.366) (end 208.28 133.35) (width 0.5) (layer F.Cu) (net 10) (status 80000))
 (segment (start 208.28 133.35) (end 207.264 132.334) (width 0.5) (layer F.Cu) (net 10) (status 80000))
 (segment (start 207.264 132.334) (end 207.264 130.302) (width 0.5) (layer F.Cu) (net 10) (status 80000))
 (segment (start 207.264 130.302) (end 207.01 130.048) (width 0.5) (layer F.Cu) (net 10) (status 80000))
 (segment (start 207.01 130.048) (end 207.01 129.032) (width 0.5) (layer F.Cu) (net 10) (status 80000))
 (segment (start 207.01 129.032) (end 207.01 127.254) (width 0.5) (layer B.Cu) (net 10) (status 80000))
 (segment (start 207.01 127.254) (end 203.2 123.444) (width 0.5) (layer B.Cu) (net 10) (status 80000))
 (segment (start 203.2 123.444) (end 203.2 122.428) (width 0.5) (layer B.Cu) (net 10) (status 80000))
 (segment (start 203.2 122.428) (end 202.438 121.666) (width 0.5) (layer B.Cu) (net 10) (status 80000))
 (segment (start 168.656 125.222) (end 170.434 125.222) (width 0.5) (layer F.Cu) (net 11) (status 80000))
 (segment (start 170.434 125.222) (end 172.466 127.254) (width 0.5) (layer F.Cu) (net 11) (status 80000))
 (segment (start 172.466 127.254) (end 172.466 149.098) (width 0.5) (layer F.Cu) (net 11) (status 80000))
 (segment (start 172.466 149.098) (end 169.672 151.892) (width 0.5) (layer F.Cu) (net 11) (status 80000))
 (segment (start 169.672 151.892) (end 169.672 152.146) (width 0.5) (layer F.Cu) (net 11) (status 80000))
 (segment (start 179.832 120.65) (end 176.53 123.952) (width 0.5) (layer F.Cu) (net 11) (status 80000))
 (segment (start 176.53 123.952) (end 175.26 125.222) (width 0.5) (layer B.Cu) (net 11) (status 80000))
 (segment (start 175.26 125.222) (end 168.656 125.222) (width 0.5) (layer B.Cu) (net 11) (status 80000))
 (segment (start 185.42 120.65) (end 179.832 120.65) (width 0.5) (layer B.Cu) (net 11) (status 80000))
 (segment (start 169.672 147.146) (end 169.672 147.066) (width 0.5) (layer F.Cu) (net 12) (status 80000))
 (segment (start 169.672 147.066) (end 166.37 150.368) (width 0.5) (layer F.Cu) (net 12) (status 80000))
 (segment (start 166.37 150.368) (end 166.37 156.21) (width 0.5) (layer F.Cu) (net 12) (status 80000))
 (segment (start 169.672 147.146) (end 169.672 142.146) (width 0.5) (layer F.Cu) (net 12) (status 80000))
 (segment (start 168.656 122.682) (end 168.91 122.428) (width 0.5) (layer B.Cu) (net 22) (status 80000))
 (segment (start 168.91 122.428) (end 186.436 122.428) (width 0.5) (layer B.Cu) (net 22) (status 80000))
 (segment (start 186.436 122.428) (end 188.214 120.65) (width 0.5) (layer B.Cu) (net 22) (status 80000))
 (segment (start 188.214 120.65) (end 190.754 120.65) (width 0.5) (layer B.Cu) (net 22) (status 80000))
 (segment (start 190.754 120.65) (end 196.088 120.65) (width 0.5) (layer B.Cu) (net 22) (status 80000))
 (segment (start 194.31 128.778) (end 193.294 129.794) (width 0.5) (layer F.Cu) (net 14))
 (segment (start 200.152 127.508) (end 200.66 127.508) (width 0.5) (layer B.Cu) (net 14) (status 80000))
 (segment (start 201.422 126.746) (end 200.66 127.508) (width 0.5) (layer B.Cu) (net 14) (status 80000))
 (segment (start 201.422 123.952) (end 201.422 126.746) (width 0.5) (layer B.Cu) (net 14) (status 80000))
 (segment (start 198.882 123.952) (end 201.422 123.952) (width 0.5) (layer B.Cu) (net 14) (status 80000))
 (segment (start 198.882 124.206) (end 198.882 123.952) (width 0.5) (layer B.Cu) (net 14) (status 80000))
 (segment (start 194.31 128.778) (end 198.882 124.206) (width 0.5) (layer B.Cu) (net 14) (status 80000))
 (segment (start 188.976 141.224) (end 188.976 137.668) (width 0.5) (layer F.Cu) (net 14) (status 80000))
 (segment (start 188.468 141.732) (end 188.976 141.224) (width 0.5) (layer F.Cu) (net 14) (status 80000))
 (segment (start 191.516 144.78) (end 188.468 141.732) (width 0.5) (layer B.Cu) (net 14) (status 80000))
 (segment (start 191.516 152.654) (end 191.516 144.78) (width 0.5) (layer F.Cu) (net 14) (status 80000))
 (segment (start 194.056 155.194) (end 191.516 152.654) (width 0.5) (layer F.Cu) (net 14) (status 80000))
 (segment (start 194.31 155.448) (end 194.056 155.194) (width 0.5) (layer B.Cu) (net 14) (status 80000))
 (segment (start 194.818 155.448) (end 194.31 155.448) (width 0.5) (layer B.Cu) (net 14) (status 80000))
 (segment (start 202.692 163.322) (end 194.818 155.448) (width 0.5) (layer B.Cu) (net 14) (status 80000))
 (segment (start 202.692 163.322) (end 202.692 165.608) (width 0.5) (layer B.Cu) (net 14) (status 80000))
 (segment (start 188.976 135.636) (end 188.976 137.668) (width 0.5) (layer F.Cu) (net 14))
 (segment (start 193.294 131.318) (end 188.976 135.636) (width 0.5) (layer F.Cu) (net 14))
 (segment (start 193.294 129.794) (end 193.294 131.318) (width 0.5) (layer F.Cu) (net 14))
 (segment (start 202.656 165.608) (end 202.692 165.608) (width 0.5) (layer B.Cu) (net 14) (status 80000))
 (segment (start 200.152 127.508) (end 200.148 127.418) (width 0.5) (layer B.Cu) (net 14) (status 80000))
 (segment (start 200.148 131.418) (end 200.152 131.318) (width 0.5) (layer B.Cu) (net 15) (status 80000))
 (segment (start 200.152 131.318) (end 200.406 131.064) (width 0.5) (layer B.Cu) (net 15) (status 80000))
 (segment (start 200.406 131.064) (end 201.93 131.064) (width 0.5) (layer B.Cu) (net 15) (status 80000))
 (segment (start 201.93 131.064) (end 200.152 132.842) (width 0.5) (layer F.Cu) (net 15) (status 80000))
 (segment (start 200.152 132.842) (end 200.152 139.954) (width 0.5) (layer F.Cu) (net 15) (status 80000))
 (segment (start 200.152 139.954) (end 202.184 141.986) (width 0.5) (layer F.Cu) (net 15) (status 80000))
 (segment (start 202.184 141.986) (end 202.184 164.338) (width 0.5) (layer F.Cu) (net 15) (status 80000))
 (segment (start 202.184 164.338) (end 200.66 165.862) (width 0.5) (layer F.Cu) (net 15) (status 80000))
 (segment (start 200.66 165.862) (end 200.66 167.64) (width 0.5) (layer F.Cu) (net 15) (status 80000))
 (segment (start 200.66 167.64) (end 200.152 167.132) (width 0.5) (layer B.Cu) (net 15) (status 80000))
 (segment (start 200.152 167.132) (end 200.152 165.608) (width 0.5) (layer B.Cu) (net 15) (status 80000))
 (segment (start 200.152 165.608) (end 200.126 165.608) (width 0.5) (layer B.Cu) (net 15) (status 80000))
 (segment (start 195.58 134.62) (end 194.564 135.636) (width 0.5) (layer B.Cu) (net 16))
 (segment (start 198.882 165.608) (end 198.882 164.084) (width 0.5) (layer B.Cu) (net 16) (status 80000))
 (segment (start 198.374 163.576) (end 198.882 164.084) (width 0.5) (layer B.Cu) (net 16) (status 80000))
 (segment (start 198.374 148.844) (end 198.374 163.576) (width 0.5) (layer F.Cu) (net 16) (status 80000))
 (segment (start 194.056 144.526) (end 198.374 148.844) (width 0.5) (layer F.Cu) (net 16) (status 80000))
 (segment (start 194.056 144.018) (end 194.056 144.526) (width 0.5) (layer F.Cu) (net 16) (status 80000))
 (segment (start 193.802 143.764) (end 194.056 144.018) (width 0.5) (layer F.Cu) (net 16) (status 80000))
 (segment (start 193.802 143.256) (end 193.802 143.764) (width 0.5) (layer F.Cu) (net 16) (status 80000))
 (segment (start 191.516 140.97) (end 193.802 143.256) (width 0.5) (layer F.Cu) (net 16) (status 80000))
 (segment (start 198.374 134.62) (end 195.58 134.62) (width 0.5) (layer B.Cu) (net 16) (status 80000))
 (segment (start 198.882 134.112) (end 198.374 134.62) (width 0.5) (layer B.Cu) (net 16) (status 80000))
 (segment (start 199.39 134.112) (end 198.882 134.112) (width 0.5) (layer B.Cu) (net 16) (status 80000))
 (segment (start 199.39 134.112) (end 200.152 133.35) (width 0.5) (layer B.Cu) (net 16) (status 80000))
 (segment (start 188.722 138.176) (end 191.516 140.97) (width 0.5) (layer B.Cu) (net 16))
 (segment (start 188.722 136.398) (end 188.722 138.176) (width 0.5) (layer B.Cu) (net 16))
 (segment (start 189.484 135.636) (end 188.722 136.398) (width 0.5) (layer B.Cu) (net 16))
 (segment (start 194.564 135.636) (end 189.484 135.636) (width 0.5) (layer B.Cu) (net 16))
 (segment (start 200.148 133.418) (end 200.152 133.35) (width 0.5) (layer B.Cu) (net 16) (status 80000))
 (segment (start 198.882 165.608) (end 198.846 165.608) (width 0.5) (layer B.Cu) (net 16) (status 80000))
 (segment (start 200.148 135.418) (end 200.152 135.382) (width 0.5) (layer B.Cu) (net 17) (status 80000))
 (segment (start 200.152 135.382) (end 199.644 135.89) (width 0.5) (layer B.Cu) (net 17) (status 80000))
 (segment (start 199.644 135.89) (end 196.342 135.89) (width 0.5) (layer B.Cu) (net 17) (status 80000))
 (segment (start 196.342 135.89) (end 194.818 137.414) (width 0.5) (layer F.Cu) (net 17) (status 80000))
 (segment (start 194.818 137.414) (end 194.818 143.51) (width 0.5) (layer F.Cu) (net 17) (status 80000))
 (segment (start 194.818 143.51) (end 200.914 149.606) (width 0.5) (layer F.Cu) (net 17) (status 80000))
 (segment (start 200.914 149.606) (end 200.914 163.576) (width 0.5) (layer F.Cu) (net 17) (status 80000))
 (segment (start 200.914 163.576) (end 201.422 164.084) (width 0.5) (layer B.Cu) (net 17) (status 80000))
 (segment (start 201.422 164.084) (end 201.422 165.608) (width 0.5) (layer B.Cu) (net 17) (status 80000))
 (segment (start 201.422 165.608) (end 201.396 165.608) (width 0.5) (layer B.Cu) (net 17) (status 80000))
 (via (at 205.74 167.64) (size 0.889) (layers F.Cu B.Cu) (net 1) (status 80000))
 (via (at 201.422 139.192) (size 0.889) (layers F.Cu B.Cu) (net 1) (status 80000))
 (via (at 214.122 126.492) (size 0.889) (layers F.Cu B.Cu) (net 1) (status 80000))
 (via (at 205.994 131.064) (size 0.889) (layers F.Cu B.Cu) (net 2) (status 80000))
 (via (at 205.994 136.652) (size 0.889) (layers F.Cu B.Cu) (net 2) (status 80000))
 (via (at 205.994 163.576) (size 0.889) (layers F.Cu B.Cu) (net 2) (status 80000))
 (via (at 203.962 136.144) (size 0.889) (layers F.Cu B.Cu) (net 2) (status 80000))
 (via (at 208.026 136.144) (size 0.889) (layers F.Cu B.Cu) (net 2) (status 80000))
 (via (at 187.452 136.144) (size 0.889) (layers F.Cu B.Cu) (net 5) (status 80000))
 (via (at 204.216 162.56) (size 0.889) (layers F.Cu B.Cu) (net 13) (status 80000))
 (via (at 203.708 146.304) (size 0.889) (layers F.Cu B.Cu) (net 13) (status 80000))
 (via (at 197.866 128.778) (size 0.889) (layers F.Cu B.Cu) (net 13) (status 80000))
 (via (at 210.312 126.238) (size 0.889) (layers F.Cu B.Cu) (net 8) (status 80000))
 (via (at 209.55 129.54) (size 0.889) (layers F.Cu B.Cu) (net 9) (status 80000))
 (via (at 212.09 163.576) (size 0.889) (layers F.Cu B.Cu) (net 10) (status 80000))
 (via (at 209.804 161.29) (size 0.889) (layers F.Cu B.Cu) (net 10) (status 80000))
 (via (at 207.01 129.032) (size 0.889) (layers F.Cu B.Cu) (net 10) (status 80000))
 (via (at 176.53 123.952) (size 0.889) (layers F.Cu B.Cu) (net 11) (status 80000))
 (via (at 194.31 128.778) (size 0.889) (layers F.Cu B.Cu) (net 14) (status 80000))
 (via (at 188.468 141.732) (size 0.889) (layers F.Cu B.Cu) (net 14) (status 80000))
 (via (at 191.516 144.78) (size 0.889) (layers F.Cu B.Cu) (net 14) (status 80000))
 (via (at 194.056 155.194) (size 0.889) (layers F.Cu B.Cu) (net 14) (status 80000))
 (via (at 201.93 131.064) (size 0.889) (layers F.Cu B.Cu) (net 15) (status 80000))
 (via (at 200.66 167.64) (size 0.889) (layers F.Cu B.Cu) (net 15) (status 80000))
 (via (at 198.374 163.576) (size 0.889) (layers F.Cu B.Cu) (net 16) (status 80000))
 (via (at 191.516 140.97) (size 0.889) (layers F.Cu B.Cu) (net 16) (status 80000))
 (via (at 196.342 135.89) (size 0.889) (layers F.Cu B.Cu) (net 17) (status 80000))
 (via (at 200.914 163.576) (size 0.889) (layers F.Cu B.Cu) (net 17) (status 80000)))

